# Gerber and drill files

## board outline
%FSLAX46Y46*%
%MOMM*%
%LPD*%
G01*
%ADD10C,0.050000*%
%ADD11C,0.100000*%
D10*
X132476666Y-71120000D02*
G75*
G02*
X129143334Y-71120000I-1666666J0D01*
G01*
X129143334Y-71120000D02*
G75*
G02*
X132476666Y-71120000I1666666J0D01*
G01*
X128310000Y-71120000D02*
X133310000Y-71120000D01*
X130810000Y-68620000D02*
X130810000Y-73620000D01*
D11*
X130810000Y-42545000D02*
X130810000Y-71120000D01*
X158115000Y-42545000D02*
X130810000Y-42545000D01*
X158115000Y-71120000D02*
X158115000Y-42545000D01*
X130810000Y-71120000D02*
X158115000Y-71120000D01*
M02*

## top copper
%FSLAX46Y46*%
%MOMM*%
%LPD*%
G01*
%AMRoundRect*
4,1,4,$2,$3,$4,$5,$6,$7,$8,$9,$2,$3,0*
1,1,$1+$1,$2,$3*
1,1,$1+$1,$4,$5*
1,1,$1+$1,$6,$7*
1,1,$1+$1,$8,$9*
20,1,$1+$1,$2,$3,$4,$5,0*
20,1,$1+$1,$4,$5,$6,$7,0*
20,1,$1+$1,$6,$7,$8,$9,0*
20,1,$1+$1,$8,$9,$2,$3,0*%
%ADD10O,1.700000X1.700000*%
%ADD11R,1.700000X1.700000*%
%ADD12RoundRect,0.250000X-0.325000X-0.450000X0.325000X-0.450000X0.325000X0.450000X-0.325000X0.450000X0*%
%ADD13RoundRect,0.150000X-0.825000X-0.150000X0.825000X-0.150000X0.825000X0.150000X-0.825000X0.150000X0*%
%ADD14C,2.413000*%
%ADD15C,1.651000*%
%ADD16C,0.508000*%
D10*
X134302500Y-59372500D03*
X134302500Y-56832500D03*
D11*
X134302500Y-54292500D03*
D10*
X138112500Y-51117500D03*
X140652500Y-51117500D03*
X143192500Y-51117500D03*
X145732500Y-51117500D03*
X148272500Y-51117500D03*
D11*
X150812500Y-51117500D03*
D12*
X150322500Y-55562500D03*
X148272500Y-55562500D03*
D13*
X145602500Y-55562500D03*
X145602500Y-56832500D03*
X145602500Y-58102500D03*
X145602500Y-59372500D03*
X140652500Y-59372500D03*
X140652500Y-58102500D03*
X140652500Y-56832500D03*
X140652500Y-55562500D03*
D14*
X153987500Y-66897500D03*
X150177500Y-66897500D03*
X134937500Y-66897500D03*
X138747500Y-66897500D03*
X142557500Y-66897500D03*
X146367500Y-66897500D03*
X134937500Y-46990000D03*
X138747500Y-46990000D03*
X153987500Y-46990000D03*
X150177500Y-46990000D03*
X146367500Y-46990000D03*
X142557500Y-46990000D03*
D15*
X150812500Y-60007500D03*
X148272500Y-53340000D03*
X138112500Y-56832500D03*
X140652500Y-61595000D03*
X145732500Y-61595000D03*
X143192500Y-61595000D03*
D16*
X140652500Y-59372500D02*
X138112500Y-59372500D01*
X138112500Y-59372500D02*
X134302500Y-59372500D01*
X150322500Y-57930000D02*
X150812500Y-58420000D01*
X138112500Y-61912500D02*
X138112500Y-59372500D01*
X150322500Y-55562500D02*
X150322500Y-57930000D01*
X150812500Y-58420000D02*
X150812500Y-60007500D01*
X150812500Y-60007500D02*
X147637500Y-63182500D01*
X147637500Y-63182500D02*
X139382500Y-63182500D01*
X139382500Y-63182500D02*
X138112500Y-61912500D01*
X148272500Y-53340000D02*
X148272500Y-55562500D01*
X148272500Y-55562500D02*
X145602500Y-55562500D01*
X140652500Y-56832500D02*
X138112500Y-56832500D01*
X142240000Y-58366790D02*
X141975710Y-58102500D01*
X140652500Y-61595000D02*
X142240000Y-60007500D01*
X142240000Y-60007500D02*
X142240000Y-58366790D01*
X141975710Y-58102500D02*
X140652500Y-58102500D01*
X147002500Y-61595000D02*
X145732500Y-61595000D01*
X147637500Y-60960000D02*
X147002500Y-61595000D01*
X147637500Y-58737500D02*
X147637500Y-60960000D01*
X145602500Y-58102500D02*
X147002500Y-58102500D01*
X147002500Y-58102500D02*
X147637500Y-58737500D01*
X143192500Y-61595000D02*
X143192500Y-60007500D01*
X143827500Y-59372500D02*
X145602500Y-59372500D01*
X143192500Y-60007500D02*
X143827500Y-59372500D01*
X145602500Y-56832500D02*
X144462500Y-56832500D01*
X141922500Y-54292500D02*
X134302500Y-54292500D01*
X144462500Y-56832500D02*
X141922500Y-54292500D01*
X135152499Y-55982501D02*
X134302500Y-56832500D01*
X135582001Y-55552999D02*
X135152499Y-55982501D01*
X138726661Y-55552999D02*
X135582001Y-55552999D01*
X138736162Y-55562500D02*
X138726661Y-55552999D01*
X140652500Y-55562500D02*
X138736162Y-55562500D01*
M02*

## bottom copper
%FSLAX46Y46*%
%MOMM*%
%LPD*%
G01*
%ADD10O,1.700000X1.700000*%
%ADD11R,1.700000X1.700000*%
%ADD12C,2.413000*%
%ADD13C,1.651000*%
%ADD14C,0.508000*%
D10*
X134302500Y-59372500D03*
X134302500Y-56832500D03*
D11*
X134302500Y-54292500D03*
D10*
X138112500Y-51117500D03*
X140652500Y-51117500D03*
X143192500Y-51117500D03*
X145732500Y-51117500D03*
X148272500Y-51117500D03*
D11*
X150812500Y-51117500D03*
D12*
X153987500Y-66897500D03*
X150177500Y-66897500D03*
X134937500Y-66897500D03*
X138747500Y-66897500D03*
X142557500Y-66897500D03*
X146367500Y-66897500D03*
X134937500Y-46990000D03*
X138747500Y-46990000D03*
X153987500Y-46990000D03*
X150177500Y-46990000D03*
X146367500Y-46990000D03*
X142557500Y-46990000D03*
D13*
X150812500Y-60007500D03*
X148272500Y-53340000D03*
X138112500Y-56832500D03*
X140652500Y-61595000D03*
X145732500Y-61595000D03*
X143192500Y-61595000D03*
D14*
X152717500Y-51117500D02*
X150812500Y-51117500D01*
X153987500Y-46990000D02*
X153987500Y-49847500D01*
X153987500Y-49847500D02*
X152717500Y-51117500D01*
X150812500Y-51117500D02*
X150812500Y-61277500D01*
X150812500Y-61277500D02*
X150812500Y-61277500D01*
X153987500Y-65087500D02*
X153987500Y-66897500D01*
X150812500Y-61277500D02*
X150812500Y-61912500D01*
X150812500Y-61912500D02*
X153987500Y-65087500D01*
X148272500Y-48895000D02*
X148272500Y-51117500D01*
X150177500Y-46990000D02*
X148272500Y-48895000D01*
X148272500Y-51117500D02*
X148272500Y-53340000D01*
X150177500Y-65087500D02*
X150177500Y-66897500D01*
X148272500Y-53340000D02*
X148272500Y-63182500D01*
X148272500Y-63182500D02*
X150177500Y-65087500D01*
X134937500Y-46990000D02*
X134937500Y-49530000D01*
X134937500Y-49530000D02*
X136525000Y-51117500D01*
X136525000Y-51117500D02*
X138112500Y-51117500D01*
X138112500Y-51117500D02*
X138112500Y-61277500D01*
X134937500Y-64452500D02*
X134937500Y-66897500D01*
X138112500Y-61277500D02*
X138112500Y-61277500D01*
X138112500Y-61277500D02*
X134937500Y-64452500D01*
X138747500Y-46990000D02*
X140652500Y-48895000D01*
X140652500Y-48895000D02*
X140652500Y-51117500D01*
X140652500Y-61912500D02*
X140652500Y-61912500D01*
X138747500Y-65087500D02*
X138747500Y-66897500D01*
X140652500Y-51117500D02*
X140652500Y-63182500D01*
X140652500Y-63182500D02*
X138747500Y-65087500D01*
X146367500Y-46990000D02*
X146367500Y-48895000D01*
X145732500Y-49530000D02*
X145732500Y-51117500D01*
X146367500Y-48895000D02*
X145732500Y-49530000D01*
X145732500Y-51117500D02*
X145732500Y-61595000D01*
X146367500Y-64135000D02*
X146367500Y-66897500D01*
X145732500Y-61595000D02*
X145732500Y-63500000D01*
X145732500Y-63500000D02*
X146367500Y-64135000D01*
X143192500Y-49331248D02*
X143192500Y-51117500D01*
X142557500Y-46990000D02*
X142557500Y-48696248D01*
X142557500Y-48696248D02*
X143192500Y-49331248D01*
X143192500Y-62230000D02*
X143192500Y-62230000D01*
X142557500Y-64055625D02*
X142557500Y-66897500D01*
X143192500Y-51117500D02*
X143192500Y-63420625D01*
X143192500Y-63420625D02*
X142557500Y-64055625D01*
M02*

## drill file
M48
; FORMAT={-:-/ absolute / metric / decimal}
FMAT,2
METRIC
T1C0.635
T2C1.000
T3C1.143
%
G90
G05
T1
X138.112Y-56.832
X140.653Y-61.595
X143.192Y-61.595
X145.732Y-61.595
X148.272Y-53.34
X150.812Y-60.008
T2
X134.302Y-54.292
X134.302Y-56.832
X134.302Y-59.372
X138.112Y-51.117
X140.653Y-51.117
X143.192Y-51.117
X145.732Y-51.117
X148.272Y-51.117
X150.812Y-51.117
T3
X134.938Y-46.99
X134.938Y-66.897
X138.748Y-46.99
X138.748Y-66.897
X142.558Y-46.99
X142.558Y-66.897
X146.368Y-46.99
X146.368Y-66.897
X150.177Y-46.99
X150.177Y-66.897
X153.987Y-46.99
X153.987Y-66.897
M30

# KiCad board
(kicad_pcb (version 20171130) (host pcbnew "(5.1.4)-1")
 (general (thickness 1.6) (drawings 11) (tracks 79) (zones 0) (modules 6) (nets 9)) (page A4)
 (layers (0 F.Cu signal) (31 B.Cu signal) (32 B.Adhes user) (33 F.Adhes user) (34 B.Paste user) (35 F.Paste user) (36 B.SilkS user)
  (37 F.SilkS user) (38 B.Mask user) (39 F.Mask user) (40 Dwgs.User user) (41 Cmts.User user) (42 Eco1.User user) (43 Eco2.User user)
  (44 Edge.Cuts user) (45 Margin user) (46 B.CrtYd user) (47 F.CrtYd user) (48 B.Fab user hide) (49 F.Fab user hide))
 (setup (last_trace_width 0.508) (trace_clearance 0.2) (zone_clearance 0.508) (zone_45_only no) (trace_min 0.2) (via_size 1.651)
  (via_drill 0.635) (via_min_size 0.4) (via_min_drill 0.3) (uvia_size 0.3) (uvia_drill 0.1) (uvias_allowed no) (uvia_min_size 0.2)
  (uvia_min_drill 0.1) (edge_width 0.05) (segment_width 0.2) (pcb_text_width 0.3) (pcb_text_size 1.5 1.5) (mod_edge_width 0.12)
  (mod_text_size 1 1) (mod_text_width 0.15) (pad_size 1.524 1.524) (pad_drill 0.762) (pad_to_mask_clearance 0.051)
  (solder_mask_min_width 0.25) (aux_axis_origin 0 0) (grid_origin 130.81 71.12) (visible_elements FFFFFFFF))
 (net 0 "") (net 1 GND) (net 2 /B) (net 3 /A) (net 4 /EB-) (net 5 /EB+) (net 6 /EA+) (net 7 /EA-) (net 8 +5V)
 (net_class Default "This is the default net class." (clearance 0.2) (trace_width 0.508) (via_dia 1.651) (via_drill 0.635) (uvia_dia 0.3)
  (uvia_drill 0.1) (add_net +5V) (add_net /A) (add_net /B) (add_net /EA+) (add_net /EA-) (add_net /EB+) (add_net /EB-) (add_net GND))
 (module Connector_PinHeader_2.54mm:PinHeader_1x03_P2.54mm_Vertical (layer F.Cu) (at 134.3025 54.2925)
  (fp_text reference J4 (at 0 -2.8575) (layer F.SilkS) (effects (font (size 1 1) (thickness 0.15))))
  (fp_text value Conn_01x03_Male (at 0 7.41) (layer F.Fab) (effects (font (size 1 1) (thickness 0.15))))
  (pad 3 thru_hole oval (at 0 5.08) (size 1.7 1.7) (drill 1) (layers *.Cu *.Mask) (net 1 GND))
  (pad 2 thru_hole oval (at 0 2.54) (size 1.7 1.7) (drill 1) (layers *.Cu *.Mask) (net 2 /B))
  (pad 1 thru_hole rect (at 0 0) (size 1.7 1.7) (drill 1) (layers *.Cu *.Mask) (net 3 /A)))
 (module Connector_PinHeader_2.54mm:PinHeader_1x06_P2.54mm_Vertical (layer F.Cu) (at 150.8125 51.1175 270)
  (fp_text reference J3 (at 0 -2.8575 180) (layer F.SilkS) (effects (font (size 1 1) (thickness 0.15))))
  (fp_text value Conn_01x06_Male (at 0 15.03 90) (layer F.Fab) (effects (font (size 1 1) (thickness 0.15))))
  (pad 6 thru_hole oval (at 0 12.7 270) (size 1.7 1.7) (drill 1) (layers *.Cu *.Mask) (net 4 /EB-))
  (pad 5 thru_hole oval (at 0 10.16 270) (size 1.7 1.7) (drill 1) (layers *.Cu *.Mask) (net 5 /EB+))
  (pad 4 thru_hole oval (at 0 7.62 270) (size 1.7 1.7) (drill 1) (layers *.Cu *.Mask) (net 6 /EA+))
  (pad 3 thru_hole oval (at 0 5.08 270) (size 1.7 1.7) (drill 1) (layers *.Cu *.Mask) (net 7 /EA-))
  (pad 2 thru_hole oval (at 0 2.54 270) (size 1.7 1.7) (drill 1) (layers *.Cu *.Mask) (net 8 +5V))
  (pad 1 thru_hole rect (at 0 0 270) (size 1.7 1.7) (drill 1) (layers *.Cu *.Mask) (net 1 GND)))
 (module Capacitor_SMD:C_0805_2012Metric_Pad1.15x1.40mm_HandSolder (layer F.Cu) (at 149.2975 55.5625)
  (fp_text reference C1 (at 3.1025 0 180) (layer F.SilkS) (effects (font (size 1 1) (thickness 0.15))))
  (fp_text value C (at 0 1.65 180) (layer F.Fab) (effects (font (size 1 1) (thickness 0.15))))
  (pad 2 smd roundrect (at 1.025 0) (size 1.15 1.4) (layers F.Cu F.Paste F.Mask) (roundrect_rratio 0.217391) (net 1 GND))
  (pad 1 smd roundrect (at -1.025 0) (size 1.15 1.4) (layers F.Cu F.Paste F.Mask) (roundrect_rratio 0.217391) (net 8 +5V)))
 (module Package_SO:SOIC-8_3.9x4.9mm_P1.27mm (layer F.Cu) (at 143.1275 57.4675)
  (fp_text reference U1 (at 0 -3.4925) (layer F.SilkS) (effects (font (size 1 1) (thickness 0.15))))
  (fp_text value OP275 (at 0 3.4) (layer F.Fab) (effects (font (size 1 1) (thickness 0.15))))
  (pad 8 smd roundrect (at 2.475 -1.905) (size 1.95 0.6) (layers F.Cu F.Paste F.Mask) (roundrect_rratio 0.25) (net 8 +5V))
  (pad 7 smd roundrect (at 2.475 -0.635) (size 1.95 0.6) (layers F.Cu F.Paste F.Mask) (roundrect_rratio 0.25) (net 3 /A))
  (pad 6 smd roundrect (at 2.475 0.635) (size 1.95 0.6) (layers F.Cu F.Paste F.Mask) (roundrect_rratio 0.25) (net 7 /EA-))
  (pad 5 smd roundrect (at 2.475 1.905) (size 1.95 0.6) (layers F.Cu F.Paste F.Mask) (roundrect_rratio 0.25) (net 6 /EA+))
  (pad 4 smd roundrect (at -2.475 1.905) (size 1.95 0.6) (layers F.Cu F.Paste F.Mask) (roundrect_rratio 0.25) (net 1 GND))
  (pad 3 smd roundrect (at -2.475 0.635) (size 1.95 0.6) (layers F.Cu F.Paste F.Mask) (roundrect_rratio 0.25) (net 5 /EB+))
  (pad 2 smd roundrect (at -2.475 -0.635) (size 1.95 0.6) (layers F.Cu F.Paste F.Mask) (roundrect_rratio 0.25) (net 4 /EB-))
  (pad 1 smd roundrect (at -2.475 -1.905) (size 1.95 0.6) (layers F.Cu F.Paste F.Mask) (roundrect_rratio 0.25) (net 2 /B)))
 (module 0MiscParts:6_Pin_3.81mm (layer F.Cu) (at 144.4625 66.8975)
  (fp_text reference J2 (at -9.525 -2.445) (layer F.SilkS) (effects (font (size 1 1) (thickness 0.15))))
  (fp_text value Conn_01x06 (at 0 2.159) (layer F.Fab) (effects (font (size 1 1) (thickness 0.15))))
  (pad 6 thru_hole circle (at 9.525 0) (size 2.413 2.413) (drill 1.143) (layers *.Cu *.Mask) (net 1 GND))
  (pad 5 thru_hole circle (at 5.715 0) (size 2.413 2.413) (drill 1.143) (layers *.Cu *.Mask) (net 8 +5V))
  (pad 1 thru_hole circle (at -9.525 0) (size 2.413 2.413) (drill 1.143) (layers *.Cu *.Mask) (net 4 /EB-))
  (pad 2 thru_hole circle (at -5.715 0) (size 2.413 2.413) (drill 1.143) (layers *.Cu *.Mask) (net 5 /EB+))
  (pad 3 thru_hole circle (at -1.905 0) (size 2.413 2.413) (drill 1.143) (layers *.Cu *.Mask) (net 6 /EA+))
  (pad 4 thru_hole circle (at 1.905 0) (size 2.413 2.413) (drill 1.143) (layers *.Cu *.Mask) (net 7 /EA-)))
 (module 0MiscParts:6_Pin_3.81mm (layer F.Cu) (at 144.4625 46.99 180)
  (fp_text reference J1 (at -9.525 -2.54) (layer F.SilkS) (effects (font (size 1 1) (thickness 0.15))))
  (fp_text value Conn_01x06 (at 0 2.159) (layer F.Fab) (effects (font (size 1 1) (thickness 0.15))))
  (pad 6 thru_hole circle (at 9.525 0 180) (size 2.413 2.413) (drill 1.143) (layers *.Cu *.Mask) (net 4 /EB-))
  (pad 5 thru_hole circle (at 5.715 0 180) (size 2.413 2.413) (drill 1.143) (layers *.Cu *.Mask) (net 5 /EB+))
  (pad 1 thru_hole circle (at -9.525 0 180) (size 2.413 2.413) (drill 1.143) (layers *.Cu *.Mask) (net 1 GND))
  (pad 2 thru_hole circle (at -5.715 0 180) (size 2.413 2.413) (drill 1.143) (layers *.Cu *.Mask) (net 8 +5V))
  (pad 3 thru_hole circle (at -1.905 0 180) (size 2.413 2.413) (drill 1.143) (layers *.Cu *.Mask) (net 7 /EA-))
  (pad 4 thru_hole circle (at 1.905 0 180) (size 2.413 2.413) (drill 1.143) (layers *.Cu *.Mask) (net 6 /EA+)))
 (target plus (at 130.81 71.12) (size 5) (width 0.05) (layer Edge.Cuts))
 (gr_line (start 130.81 42.545) (end 130.81 71.12) (layer Edge.Cuts) (width 0.1))
 (gr_line (start 158.115 42.545) (end 130.81 42.545) (layer Edge.Cuts) (width 0.1))
 (gr_line (start 158.115 71.12) (end 158.115 42.545) (layer Edge.Cuts) (width 0.1))
 (gr_line (start 130.81 71.12) (end 158.115 71.12) (layer Edge.Cuts) (width 0.1))
 (segment (start 152.7175 51.1175) (end 150.8125 51.1175) (width 0.508) (layer B.Cu) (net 1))
 (segment (start 153.9875 46.99) (end 153.9875 49.8475) (width 0.508) (layer B.Cu) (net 1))
 (segment (start 153.9875 49.8475) (end 152.7175 51.1175) (width 0.508) (layer B.Cu) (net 1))
 (segment (start 150.8125 51.1175) (end 150.8125 61.2775) (width 0.508) (layer B.Cu) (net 1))
 (segment (start 150.8125 61.2775) (end 150.8125 61.2775) (width 0.508) (layer B.Cu) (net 1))
 (via (at 150.8125 60.0075) (size 1.651) (drill 0.635) (layers F.Cu B.Cu) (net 1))
 (segment (start 140.6525 59.3725) (end 138.1125 59.3725) (width 0.508) (layer F.Cu) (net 1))
 (segment (start 138.1125 59.3725) (end 134.3025 59.3725) (width 0.508) (layer F.Cu) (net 1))
 (segment (start 153.9875 65.0875) (end 153.9875 66.8975) (width 0.508) (layer B.Cu) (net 1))
 (segment (start 150.8125 61.2775) (end 150.8125 61.9125) (width 0.508) (layer B.Cu) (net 1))
 (segment (start 150.8125 61.9125) (end 153.9875 65.0875) (width 0.508) (layer B.Cu) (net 1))
 (segment (start 150.3225 57.93) (end 150.8125 58.42) (width 0.508) (layer F.Cu) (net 1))
 (segment (start 138.1125 61.9125) (end 138.1125 59.3725) (width 0.508) (layer F.Cu) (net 1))
 (segment (start 150.3225 55.5625) (end 150.3225 57.93) (width 0.508) (layer F.Cu) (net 1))
 (segment (start 150.8125 58.42) (end 150.8125 60.0075) (width 0.508) (layer F.Cu) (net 1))
 (segment (start 150.8125 60.0075) (end 147.6375 63.1825) (width 0.508) (layer F.Cu) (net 1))
 (segment (start 147.6375 63.1825) (end 139.3825 63.1825) (width 0.508) (layer F.Cu) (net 1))
 (segment (start 139.3825 63.1825) (end 138.1125 61.9125) (width 0.508) (layer F.Cu) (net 1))
 (segment (start 148.2725 48.895) (end 148.2725 51.1175) (width 0.508) (layer B.Cu) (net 8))
 (segment (start 150.1775 46.99) (end 148.2725 48.895) (width 0.508) (layer B.Cu) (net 8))
 (segment (start 148.2725 51.1175) (end 148.2725 53.34) (width 0.508) (layer B.Cu) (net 8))
 (via (at 148.2725 53.34) (size 1.651) (drill 0.635) (layers F.Cu B.Cu) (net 8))
 (segment (start 148.2725 53.34) (end 148.2725 55.5625) (width 0.508) (layer F.Cu) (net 8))
 (segment (start 148.2725 55.5625) (end 145.6025 55.5625) (width 0.508) (layer F.Cu) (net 8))
 (segment (start 150.1775 65.0875) (end 150.1775 66.8975) (width 0.508) (layer B.Cu) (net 8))
 (segment (start 148.2725 53.34) (end 148.2725 63.1825) (width 0.508) (layer B.Cu) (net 8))
 (segment (start 148.2725 63.1825) (end 150.1775 65.0875) (width 0.508) (layer B.Cu) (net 8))
 (segment (start 134.9375 46.99) (end 134.9375 49.53) (width 0.508) (layer B.Cu) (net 4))
 (segment (start 134.9375 49.53) (end 136.525 51.1175) (width 0.508) (layer B.Cu) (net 4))
 (segment (start 136.525 51.1175) (end 138.1125 51.1175) (width 0.508) (layer B.Cu) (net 4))
 (segment (start 138.1125 51.1175) (end 138.1125 61.2775) (width 0.508) (layer B.Cu) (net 4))
 (segment (start 134.9375 64.4525) (end 134.9375 66.8975) (width 0.508) (layer B.Cu) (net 4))
 (segment (start 138.1125 61.2775) (end 138.1125 61.2775) (width 0.508) (layer B.Cu) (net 4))
 (segment (start 138.1125 61.2775) (end 134.9375 64.4525) (width 0.508) (layer B.Cu) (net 4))
 (via (at 138.1125 56.8325) (size 1.651) (drill 0.635) (layers F.Cu B.Cu) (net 4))
 (segment (start 140.6525 56.8325) (end 138.1125 56.8325) (width 0.508) (layer F.Cu) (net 4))
 (segment (start 138.7475 46.99) (end 140.6525 48.895) (width 0.508) (layer B.Cu) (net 5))
 (segment (start 140.6525 48.895) (end 140.6525 51.1175) (width 0.508) (layer B.Cu) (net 5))
 (segment (start 140.6525 61.9125) (end 140.6525 61.9125) (width 0.508) (layer B.Cu) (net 5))
 (via (at 140.6525 61.595) (size 1.651) (drill 0.635) (layers F.Cu B.Cu) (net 5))
 (segment (start 142.24 58.36679) (end 141.97571 58.1025) (width 0.508) (layer F.Cu) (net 5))
 (segment (start 140.6525 61.595) (end 142.24 60.0075) (width 0.508) (layer F.Cu) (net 5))
 (segment (start 142.24 60.0075) (end 142.24 58.36679) (width 0.508) (layer F.Cu) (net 5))
 (segment (start 141.97571 58.1025) (end 140.6525 58.1025) (width 0.508) (layer F.Cu) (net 5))
 (segment (start 138.7475 65.0875) (end 138.7475 66.8975) (width 0.508) (layer B.Cu) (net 5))
 (segment (start 140.6525 51.1175) (end 140.6525 63.1825) (width 0.508) (layer B.Cu) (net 5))
 (segment (start 140.6525 63.1825) (end 138.7475 65.0875) (width 0.508) (layer B.Cu) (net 5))
 (segment (start 146.3675 46.99) (end 146.3675 48.895) (width 0.508) (layer B.Cu) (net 7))
 (segment (start 145.7325 49.53) (end 145.7325 51.1175) (width 0.508) (layer B.Cu) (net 7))
 (segment (start 146.3675 48.895) (end 145.7325 49.53) (width 0.508) (layer B.Cu) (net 7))
 (segment (start 145.7325 51.1175) (end 145.7325 61.595) (width 0.508) (layer B.Cu) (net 7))
 (via (at 145.7325 61.595) (size 1.651) (drill 0.635) (layers F.Cu B.Cu) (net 7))
 (segment (start 147.0025 61.595) (end 145.7325 61.595) (width 0.508) (layer F.Cu) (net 7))
 (segment (start 147.6375 60.96) (end 147.0025 61.595) (width 0.508) (layer F.Cu) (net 7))
 (segment (start 147.6375 58.7375) (end 147.6375 60.96) (width 0.508) (layer F.Cu) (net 7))
 (segment (start 145.6025 58.1025) (end 147.0025 58.1025) (width 0.508) (layer F.Cu) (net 7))
 (segment (start 147.0025 58.1025) (end 147.6375 58.7375) (width 0.508) (layer F.Cu) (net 7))
 (segment (start 146.3675 64.135) (end 146.3675 66.8975) (width 0.508) (layer B.Cu) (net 7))
 (segment (start 145.7325 61.595) (end 145.7325 63.5) (width 0.508) (layer B.Cu) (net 7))
 (segment (start 145.7325 63.5) (end 146.3675 64.135) (width 0.508) (layer B.Cu) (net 7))
 (segment (start 143.1925 49.331248) (end 143.1925 51.1175) (width 0.508) (layer B.Cu) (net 6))
 (segment (start 142.5575 46.99) (end 142.5575 48.696248) (width 0.508) (layer B.Cu) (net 6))
 (segment (start 142.5575 48.696248) (end 143.1925 49.331248) (width 0.508) (layer B.Cu) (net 6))
 (segment (start 143.1925 62.23) (end 143.1925 62.23) (width 0.508) (layer B.Cu) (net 6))
 (via (at 143.1925 61.595) (size 1.651) (drill 0.635) (layers F.Cu B.Cu) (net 6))
 (segment (start 143.1925 61.595) (end 143.1925 60.0075) (width 0.508) (layer F.Cu) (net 6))
 (segment (start 143.8275 59.3725) (end 145.6025 59.3725) (width 0.508) (layer F.Cu) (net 6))
 (segment (start 143.1925 60.0075) (end 143.8275 59.3725) (width 0.508) (layer F.Cu) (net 6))
 (segment (start 142.5575 64.055625) (end 142.5575 66.8975) (width 0.508) (layer B.Cu) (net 6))
 (segment (start 143.1925 51.1175) (end 143.1925 63.420625) (width 0.508) (layer B.Cu) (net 6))
 (segment (start 143.1925 63.420625) (end 142.5575 64.055625) (width 0.508) (layer B.Cu) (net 6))
 (segment (start 145.6025 56.8325) (end 144.4625 56.8325) (width 0.508) (layer F.Cu) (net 3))
 (segment (start 141.9225 54.2925) (end 134.3025 54.2925) (width 0.508) (layer F.Cu) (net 3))
 (segment (start 144.4625 56.8325) (end 141.9225 54.2925) (width 0.508) (layer F.Cu) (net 3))
 (segment (start 135.152499 55.982501) (end 134.3025 56.8325) (width 0.508) (layer F.Cu) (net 2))
 (segment (start 135.582001 55.552999) (end 135.152499 55.982501) (width 0.508) (layer F.Cu) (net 2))
 (segment (start 138.726661 55.552999) (end 135.582001 55.552999) (width 0.508) (layer F.Cu) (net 2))
 (segment (start 138.736162 55.5625) (end 138.726661 55.552999) (width 0.508) (layer F.Cu) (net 2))
 (segment (start 140.6525 55.5625) (end 138.736162 55.5625) (width 0.508) (layer F.Cu) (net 2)))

